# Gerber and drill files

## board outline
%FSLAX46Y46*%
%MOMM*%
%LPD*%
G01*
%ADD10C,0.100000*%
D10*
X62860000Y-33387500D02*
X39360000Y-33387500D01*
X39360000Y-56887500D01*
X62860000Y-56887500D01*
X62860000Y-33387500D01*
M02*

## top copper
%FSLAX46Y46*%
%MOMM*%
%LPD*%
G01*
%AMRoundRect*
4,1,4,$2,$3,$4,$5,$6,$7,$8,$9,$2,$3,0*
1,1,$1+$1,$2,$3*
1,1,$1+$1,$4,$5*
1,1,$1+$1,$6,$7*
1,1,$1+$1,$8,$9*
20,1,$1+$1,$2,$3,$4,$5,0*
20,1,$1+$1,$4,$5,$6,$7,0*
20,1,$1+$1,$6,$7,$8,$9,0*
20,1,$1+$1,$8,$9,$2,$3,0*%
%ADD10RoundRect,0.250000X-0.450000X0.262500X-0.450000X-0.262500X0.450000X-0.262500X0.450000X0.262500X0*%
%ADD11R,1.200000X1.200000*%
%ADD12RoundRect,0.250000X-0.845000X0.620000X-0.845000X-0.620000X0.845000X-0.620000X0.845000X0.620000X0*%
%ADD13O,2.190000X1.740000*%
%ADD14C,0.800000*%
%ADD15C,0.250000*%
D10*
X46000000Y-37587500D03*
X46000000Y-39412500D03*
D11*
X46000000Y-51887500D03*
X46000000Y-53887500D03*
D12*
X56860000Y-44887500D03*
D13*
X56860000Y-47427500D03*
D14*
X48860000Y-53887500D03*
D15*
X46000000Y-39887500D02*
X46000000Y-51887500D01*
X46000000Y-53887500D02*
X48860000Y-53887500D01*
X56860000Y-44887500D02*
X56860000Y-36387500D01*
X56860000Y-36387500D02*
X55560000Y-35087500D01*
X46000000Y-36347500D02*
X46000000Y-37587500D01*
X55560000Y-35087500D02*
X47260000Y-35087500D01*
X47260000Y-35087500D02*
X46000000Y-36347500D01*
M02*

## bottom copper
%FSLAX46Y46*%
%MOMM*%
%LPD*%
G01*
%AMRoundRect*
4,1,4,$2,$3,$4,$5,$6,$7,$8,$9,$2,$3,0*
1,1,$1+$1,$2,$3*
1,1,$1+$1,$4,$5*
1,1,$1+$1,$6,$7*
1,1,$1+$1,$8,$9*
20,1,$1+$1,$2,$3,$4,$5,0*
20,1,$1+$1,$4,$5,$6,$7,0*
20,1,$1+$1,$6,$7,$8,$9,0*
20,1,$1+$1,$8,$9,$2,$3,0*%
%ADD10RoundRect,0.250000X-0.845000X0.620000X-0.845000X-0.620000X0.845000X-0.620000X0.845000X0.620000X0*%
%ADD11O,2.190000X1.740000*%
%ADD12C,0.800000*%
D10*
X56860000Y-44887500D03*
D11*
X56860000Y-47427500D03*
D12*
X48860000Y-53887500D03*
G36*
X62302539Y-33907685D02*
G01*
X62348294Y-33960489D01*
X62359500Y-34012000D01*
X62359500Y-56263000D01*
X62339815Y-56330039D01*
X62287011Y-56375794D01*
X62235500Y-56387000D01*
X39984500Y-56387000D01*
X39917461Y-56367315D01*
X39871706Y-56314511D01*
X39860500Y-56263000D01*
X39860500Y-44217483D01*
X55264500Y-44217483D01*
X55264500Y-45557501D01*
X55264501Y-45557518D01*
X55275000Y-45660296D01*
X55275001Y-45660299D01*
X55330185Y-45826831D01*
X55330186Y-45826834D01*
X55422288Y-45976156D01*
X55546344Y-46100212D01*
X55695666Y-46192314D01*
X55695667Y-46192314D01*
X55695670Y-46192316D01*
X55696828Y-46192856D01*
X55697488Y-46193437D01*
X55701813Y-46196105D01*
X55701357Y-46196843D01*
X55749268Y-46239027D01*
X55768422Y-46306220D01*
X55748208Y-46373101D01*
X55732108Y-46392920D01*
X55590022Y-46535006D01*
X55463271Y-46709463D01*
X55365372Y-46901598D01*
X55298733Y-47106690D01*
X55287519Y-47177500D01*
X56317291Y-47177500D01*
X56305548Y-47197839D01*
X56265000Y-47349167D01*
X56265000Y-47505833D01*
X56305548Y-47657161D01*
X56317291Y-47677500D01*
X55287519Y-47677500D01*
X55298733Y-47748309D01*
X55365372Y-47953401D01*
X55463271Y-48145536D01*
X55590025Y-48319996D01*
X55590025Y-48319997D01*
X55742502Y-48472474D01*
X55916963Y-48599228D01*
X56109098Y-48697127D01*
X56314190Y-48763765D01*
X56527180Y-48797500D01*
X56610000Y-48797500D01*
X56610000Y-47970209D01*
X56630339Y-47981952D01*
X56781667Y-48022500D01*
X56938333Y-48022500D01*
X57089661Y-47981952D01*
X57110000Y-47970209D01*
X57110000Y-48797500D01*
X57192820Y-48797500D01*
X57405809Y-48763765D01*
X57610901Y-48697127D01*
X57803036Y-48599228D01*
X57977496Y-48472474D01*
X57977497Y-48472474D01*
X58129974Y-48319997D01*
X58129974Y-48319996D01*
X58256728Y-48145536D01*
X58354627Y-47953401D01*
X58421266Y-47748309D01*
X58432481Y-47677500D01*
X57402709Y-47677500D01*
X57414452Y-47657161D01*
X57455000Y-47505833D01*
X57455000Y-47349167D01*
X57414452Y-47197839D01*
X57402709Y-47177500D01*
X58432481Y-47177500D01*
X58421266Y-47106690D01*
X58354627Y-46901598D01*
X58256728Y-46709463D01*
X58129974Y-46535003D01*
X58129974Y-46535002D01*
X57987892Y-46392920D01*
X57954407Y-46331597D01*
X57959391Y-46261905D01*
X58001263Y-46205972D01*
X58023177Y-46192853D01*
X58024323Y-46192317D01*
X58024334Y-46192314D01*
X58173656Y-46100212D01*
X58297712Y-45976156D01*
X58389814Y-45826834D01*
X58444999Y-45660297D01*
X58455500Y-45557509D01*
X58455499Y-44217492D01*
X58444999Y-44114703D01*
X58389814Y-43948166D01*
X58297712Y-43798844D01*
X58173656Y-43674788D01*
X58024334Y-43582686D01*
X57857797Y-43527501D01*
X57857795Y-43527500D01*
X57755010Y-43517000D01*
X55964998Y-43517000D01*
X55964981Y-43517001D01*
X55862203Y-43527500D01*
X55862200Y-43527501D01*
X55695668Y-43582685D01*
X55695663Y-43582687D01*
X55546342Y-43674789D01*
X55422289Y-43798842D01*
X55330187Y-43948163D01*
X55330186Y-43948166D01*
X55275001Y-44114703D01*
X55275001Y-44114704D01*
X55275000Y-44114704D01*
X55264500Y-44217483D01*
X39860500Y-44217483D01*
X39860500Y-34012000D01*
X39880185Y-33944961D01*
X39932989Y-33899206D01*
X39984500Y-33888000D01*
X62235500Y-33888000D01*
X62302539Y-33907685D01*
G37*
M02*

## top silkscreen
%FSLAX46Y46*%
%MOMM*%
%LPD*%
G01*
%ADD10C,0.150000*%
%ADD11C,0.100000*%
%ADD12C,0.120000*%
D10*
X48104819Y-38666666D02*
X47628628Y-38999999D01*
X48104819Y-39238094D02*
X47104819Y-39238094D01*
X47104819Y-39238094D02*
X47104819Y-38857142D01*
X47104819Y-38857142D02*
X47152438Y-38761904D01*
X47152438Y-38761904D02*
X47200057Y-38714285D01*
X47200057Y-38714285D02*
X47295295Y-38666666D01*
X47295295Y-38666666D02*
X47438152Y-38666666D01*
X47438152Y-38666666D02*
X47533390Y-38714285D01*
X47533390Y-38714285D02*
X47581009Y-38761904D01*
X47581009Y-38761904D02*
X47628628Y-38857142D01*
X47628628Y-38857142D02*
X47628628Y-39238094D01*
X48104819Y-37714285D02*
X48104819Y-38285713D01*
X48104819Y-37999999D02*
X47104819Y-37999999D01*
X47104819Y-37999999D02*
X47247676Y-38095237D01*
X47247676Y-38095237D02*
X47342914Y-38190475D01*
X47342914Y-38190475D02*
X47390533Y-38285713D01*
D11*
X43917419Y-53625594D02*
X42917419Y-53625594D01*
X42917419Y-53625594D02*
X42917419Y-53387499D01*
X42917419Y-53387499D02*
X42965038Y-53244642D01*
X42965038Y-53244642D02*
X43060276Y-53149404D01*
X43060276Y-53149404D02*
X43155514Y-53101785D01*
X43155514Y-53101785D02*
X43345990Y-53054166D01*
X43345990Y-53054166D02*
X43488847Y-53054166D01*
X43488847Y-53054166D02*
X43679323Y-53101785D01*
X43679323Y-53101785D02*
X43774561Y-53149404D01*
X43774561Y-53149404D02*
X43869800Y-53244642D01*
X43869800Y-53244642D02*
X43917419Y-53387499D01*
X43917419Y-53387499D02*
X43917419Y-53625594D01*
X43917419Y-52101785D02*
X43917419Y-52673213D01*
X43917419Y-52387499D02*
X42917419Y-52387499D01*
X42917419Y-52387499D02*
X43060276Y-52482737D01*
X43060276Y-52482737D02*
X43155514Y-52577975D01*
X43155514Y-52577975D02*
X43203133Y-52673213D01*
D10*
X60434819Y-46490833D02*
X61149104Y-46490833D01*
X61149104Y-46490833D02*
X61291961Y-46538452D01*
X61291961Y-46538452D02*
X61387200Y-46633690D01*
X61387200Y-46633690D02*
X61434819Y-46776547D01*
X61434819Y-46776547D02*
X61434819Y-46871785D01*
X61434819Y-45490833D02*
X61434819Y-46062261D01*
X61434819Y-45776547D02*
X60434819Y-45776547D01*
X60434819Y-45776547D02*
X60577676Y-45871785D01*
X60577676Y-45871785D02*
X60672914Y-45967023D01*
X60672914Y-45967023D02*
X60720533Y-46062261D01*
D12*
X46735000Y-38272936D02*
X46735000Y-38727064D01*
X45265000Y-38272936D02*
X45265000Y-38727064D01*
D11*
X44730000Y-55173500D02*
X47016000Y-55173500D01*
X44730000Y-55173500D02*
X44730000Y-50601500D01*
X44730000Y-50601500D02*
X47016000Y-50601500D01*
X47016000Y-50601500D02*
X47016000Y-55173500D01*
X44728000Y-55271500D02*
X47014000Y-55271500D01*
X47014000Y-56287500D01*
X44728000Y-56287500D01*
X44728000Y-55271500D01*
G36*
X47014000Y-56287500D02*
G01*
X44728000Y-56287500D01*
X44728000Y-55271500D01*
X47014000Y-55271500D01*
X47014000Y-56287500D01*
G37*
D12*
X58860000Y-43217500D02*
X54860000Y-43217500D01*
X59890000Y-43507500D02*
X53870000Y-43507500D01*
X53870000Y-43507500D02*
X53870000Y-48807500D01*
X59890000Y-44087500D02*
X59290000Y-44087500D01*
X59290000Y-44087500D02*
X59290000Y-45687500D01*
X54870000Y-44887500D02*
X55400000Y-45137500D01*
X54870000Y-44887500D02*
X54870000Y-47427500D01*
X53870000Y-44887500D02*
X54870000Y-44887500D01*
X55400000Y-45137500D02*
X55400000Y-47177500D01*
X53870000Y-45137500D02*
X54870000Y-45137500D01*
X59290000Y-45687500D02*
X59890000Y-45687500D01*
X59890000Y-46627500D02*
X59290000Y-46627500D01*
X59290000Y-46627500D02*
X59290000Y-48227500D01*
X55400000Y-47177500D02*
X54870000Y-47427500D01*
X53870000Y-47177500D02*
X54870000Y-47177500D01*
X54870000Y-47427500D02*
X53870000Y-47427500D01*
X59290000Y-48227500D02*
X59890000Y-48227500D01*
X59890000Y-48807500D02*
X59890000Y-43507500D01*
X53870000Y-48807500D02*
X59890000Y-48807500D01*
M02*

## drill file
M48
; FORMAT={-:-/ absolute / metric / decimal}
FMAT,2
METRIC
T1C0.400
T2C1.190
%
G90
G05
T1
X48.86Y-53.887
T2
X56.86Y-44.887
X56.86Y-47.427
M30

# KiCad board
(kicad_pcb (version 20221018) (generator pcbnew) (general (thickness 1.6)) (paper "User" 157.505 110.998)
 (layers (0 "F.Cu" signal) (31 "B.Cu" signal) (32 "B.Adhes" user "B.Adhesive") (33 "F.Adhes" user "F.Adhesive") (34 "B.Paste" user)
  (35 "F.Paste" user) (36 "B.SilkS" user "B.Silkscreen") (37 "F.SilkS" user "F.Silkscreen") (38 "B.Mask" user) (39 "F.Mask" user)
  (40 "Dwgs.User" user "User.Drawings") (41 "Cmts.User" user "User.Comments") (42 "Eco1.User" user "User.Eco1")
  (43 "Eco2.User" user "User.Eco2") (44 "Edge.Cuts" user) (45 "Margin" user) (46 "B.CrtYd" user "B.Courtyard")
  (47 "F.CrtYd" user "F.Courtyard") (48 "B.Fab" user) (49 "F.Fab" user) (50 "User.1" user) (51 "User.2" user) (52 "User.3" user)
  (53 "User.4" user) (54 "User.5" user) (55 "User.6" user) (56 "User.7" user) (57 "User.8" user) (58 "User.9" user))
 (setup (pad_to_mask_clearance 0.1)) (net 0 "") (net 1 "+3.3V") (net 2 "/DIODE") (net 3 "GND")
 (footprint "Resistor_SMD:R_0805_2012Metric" (layer "F.Cu") (at 46 38.5 -90)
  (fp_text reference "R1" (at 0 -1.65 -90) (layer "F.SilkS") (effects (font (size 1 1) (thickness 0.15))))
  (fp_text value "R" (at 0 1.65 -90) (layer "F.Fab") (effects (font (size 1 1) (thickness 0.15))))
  (fp_line (start -0.227064 -0.735) (end 0.227064 -0.735) (stroke (width 0.12) (type solid)) (layer "F.SilkS"))
  (fp_line (start -0.227064 0.735) (end 0.227064 0.735) (stroke (width 0.12) (type solid)) (layer "F.SilkS"))
  (pad "1" smd roundrect (at -0.9125 0 270) (size 1.025 1.4) (layers "F.Cu" "F.Paste" "F.Mask") (roundrect_rratio 0.243902439)
   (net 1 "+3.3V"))
  (pad "2" smd roundrect (at 0.9125 0 270) (size 1.025 1.4) (layers "F.Cu" "F.Paste" "F.Mask") (roundrect_rratio 0.243902439)
   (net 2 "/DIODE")))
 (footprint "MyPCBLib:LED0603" (layer "F.Cu") (at 46 52.8875 90)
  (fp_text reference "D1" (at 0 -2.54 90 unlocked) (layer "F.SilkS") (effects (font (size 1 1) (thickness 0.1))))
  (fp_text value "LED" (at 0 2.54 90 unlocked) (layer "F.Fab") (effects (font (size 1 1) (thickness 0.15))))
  (fp_line (start -2.286 -1.27) (end -2.286 1.016) (stroke (width 0.1) (type default)) (layer "F.SilkS"))
  (fp_line (start -2.286 -1.27) (end 2.286 -1.27) (stroke (width 0.1) (type default)) (layer "F.SilkS"))
  (fp_line (start 2.286 -1.27) (end 2.286 1.016) (stroke (width 0.1) (type default)) (layer "F.SilkS"))
  (fp_line (start 2.286 1.016) (end -2.286 1.016) (stroke (width 0.1) (type default)) (layer "F.SilkS"))
  (fp_poly
   (pts (xy -2.384 -1.272) (xy -2.384 1.014) (xy -3.4 1.014) (xy -3.4 -1.272)) (stroke (width 0.1) (type solid)) (fill solid)
   (layer "F.SilkS"))
  (pad "A" smd rect (at 1 0 90) (size 1.2 1.2) (layers "F.Cu" "F.Paste" "F.Mask") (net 2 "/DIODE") (thermal_bridge_angle 45))
  (pad "C" smd rect (at -1 0 90) (size 1.2 1.2) (layers "F.Cu" "F.Paste" "F.Mask") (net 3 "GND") (thermal_bridge_angle 45)))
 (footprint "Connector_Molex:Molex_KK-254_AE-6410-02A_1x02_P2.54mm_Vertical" (layer "F.Cu") (at 56.86 44.8875 -90)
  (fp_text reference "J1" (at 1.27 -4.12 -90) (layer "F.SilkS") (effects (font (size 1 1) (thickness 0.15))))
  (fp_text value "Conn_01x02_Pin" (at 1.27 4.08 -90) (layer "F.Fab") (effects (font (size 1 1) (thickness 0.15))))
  (fp_line (start -1.67 -2) (end -1.67 2) (stroke (width 0.12) (type solid)) (layer "F.SilkS"))
  (fp_line (start -1.38 -3.03) (end -1.38 2.99) (stroke (width 0.12) (type solid)) (layer "F.SilkS"))
  (fp_line (start -1.38 2.99) (end 3.92 2.99) (stroke (width 0.12) (type solid)) (layer "F.SilkS"))
  (fp_line (start -0.8 -3.03) (end -0.8 -2.43) (stroke (width 0.12) (type solid)) (layer "F.SilkS"))
  (fp_line (start -0.8 -2.43) (end 0.8 -2.43) (stroke (width 0.12) (type solid)) (layer "F.SilkS"))
  (fp_line (start 0 1.99) (end 0.25 1.46) (stroke (width 0.12) (type solid)) (layer "F.SilkS"))
  (fp_line (start 0 1.99) (end 2.54 1.99) (stroke (width 0.12) (type solid)) (layer "F.SilkS"))
  (fp_line (start 0 2.99) (end 0 1.99) (stroke (width 0.12) (type solid)) (layer "F.SilkS"))
  (fp_line (start 0.25 1.46) (end 2.29 1.46) (stroke (width 0.12) (type solid)) (layer "F.SilkS"))
  (fp_line (start 0.25 2.99) (end 0.25 1.99) (stroke (width 0.12) (type solid)) (layer "F.SilkS"))
  (fp_line (start 0.8 -2.43) (end 0.8 -3.03) (stroke (width 0.12) (type solid)) (layer "F.SilkS"))
  (fp_line (start 1.74 -3.03) (end 1.74 -2.43) (stroke (width 0.12) (type solid)) (layer "F.SilkS"))
  (fp_line (start 1.74 -2.43) (end 3.34 -2.43) (stroke (width 0.12) (type solid)) (layer "F.SilkS"))
  (fp_line (start 2.29 1.46) (end 2.54 1.99) (stroke (width 0.12) (type solid)) (layer "F.SilkS"))
  (fp_line (start 2.29 2.99) (end 2.29 1.99) (stroke (width 0.12) (type solid)) (layer "F.SilkS"))
  (fp_line (start 2.54 1.99) (end 2.54 2.99) (stroke (width 0.12) (type solid)) (layer "F.SilkS"))
  (fp_line (start 3.34 -2.43) (end 3.34 -3.03) (stroke (width 0.12) (type solid)) (layer "F.SilkS"))
  (fp_line (start 3.92 -3.03) (end -1.38 -3.03) (stroke (width 0.12) (type solid)) (layer "F.SilkS"))
  (fp_line (start 3.92 2.99) (end 3.92 -3.03) (stroke (width 0.12) (type solid)) (layer "F.SilkS"))
  (pad "1" thru_hole roundrect (at 0 0 270) (size 1.74 2.19) (drill 1.19) (layers "*.Cu" "*.Mask") (roundrect_rratio 0.1436781609)
   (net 1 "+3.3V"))
  (pad "2" thru_hole oval (at 2.54 0 270) (size 1.74 2.19) (drill 1.19) (layers "*.Cu" "*.Mask") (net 3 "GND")))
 (gr_poly
  (pts (xy 62.86 33.3875) (xy 39.36 33.3875) (xy 39.36 56.8875) (xy 62.86 56.8875)) (stroke (width 0.1) (type solid)) (fill none)
  (layer "Edge.Cuts"))
 (segment (start 46 39.8875) (end 46 51.8875) (width 0.25) (layer "F.Cu") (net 2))
 (segment (start 46 53.8875) (end 48.86 53.8875) (width 0.25) (layer "F.Cu") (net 3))
 (via (at 48.86 53.8875) (size 0.8) (drill 0.4) (layers "F.Cu" "B.Cu") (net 3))
 (segment (start 56.86 44.8875) (end 56.86 36.3875) (width 0.25) (layer "F.Cu") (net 1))
 (segment (start 56.86 36.3875) (end 55.56 35.0875) (width 0.25) (layer "F.Cu") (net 1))
 (segment (start 46 36.3475) (end 46 37.5875) (width 0.25) (layer "F.Cu") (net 1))
 (segment (start 55.56 35.0875) (end 47.26 35.0875) (width 0.25) (layer "F.Cu") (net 1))
 (segment (start 47.26 35.0875) (end 46 36.3475) (width 0.25) (layer "F.Cu") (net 1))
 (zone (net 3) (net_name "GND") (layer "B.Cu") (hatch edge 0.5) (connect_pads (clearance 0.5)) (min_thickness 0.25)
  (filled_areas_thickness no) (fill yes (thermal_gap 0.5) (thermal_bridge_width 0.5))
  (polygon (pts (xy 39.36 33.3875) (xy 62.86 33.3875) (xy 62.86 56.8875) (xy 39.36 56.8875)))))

